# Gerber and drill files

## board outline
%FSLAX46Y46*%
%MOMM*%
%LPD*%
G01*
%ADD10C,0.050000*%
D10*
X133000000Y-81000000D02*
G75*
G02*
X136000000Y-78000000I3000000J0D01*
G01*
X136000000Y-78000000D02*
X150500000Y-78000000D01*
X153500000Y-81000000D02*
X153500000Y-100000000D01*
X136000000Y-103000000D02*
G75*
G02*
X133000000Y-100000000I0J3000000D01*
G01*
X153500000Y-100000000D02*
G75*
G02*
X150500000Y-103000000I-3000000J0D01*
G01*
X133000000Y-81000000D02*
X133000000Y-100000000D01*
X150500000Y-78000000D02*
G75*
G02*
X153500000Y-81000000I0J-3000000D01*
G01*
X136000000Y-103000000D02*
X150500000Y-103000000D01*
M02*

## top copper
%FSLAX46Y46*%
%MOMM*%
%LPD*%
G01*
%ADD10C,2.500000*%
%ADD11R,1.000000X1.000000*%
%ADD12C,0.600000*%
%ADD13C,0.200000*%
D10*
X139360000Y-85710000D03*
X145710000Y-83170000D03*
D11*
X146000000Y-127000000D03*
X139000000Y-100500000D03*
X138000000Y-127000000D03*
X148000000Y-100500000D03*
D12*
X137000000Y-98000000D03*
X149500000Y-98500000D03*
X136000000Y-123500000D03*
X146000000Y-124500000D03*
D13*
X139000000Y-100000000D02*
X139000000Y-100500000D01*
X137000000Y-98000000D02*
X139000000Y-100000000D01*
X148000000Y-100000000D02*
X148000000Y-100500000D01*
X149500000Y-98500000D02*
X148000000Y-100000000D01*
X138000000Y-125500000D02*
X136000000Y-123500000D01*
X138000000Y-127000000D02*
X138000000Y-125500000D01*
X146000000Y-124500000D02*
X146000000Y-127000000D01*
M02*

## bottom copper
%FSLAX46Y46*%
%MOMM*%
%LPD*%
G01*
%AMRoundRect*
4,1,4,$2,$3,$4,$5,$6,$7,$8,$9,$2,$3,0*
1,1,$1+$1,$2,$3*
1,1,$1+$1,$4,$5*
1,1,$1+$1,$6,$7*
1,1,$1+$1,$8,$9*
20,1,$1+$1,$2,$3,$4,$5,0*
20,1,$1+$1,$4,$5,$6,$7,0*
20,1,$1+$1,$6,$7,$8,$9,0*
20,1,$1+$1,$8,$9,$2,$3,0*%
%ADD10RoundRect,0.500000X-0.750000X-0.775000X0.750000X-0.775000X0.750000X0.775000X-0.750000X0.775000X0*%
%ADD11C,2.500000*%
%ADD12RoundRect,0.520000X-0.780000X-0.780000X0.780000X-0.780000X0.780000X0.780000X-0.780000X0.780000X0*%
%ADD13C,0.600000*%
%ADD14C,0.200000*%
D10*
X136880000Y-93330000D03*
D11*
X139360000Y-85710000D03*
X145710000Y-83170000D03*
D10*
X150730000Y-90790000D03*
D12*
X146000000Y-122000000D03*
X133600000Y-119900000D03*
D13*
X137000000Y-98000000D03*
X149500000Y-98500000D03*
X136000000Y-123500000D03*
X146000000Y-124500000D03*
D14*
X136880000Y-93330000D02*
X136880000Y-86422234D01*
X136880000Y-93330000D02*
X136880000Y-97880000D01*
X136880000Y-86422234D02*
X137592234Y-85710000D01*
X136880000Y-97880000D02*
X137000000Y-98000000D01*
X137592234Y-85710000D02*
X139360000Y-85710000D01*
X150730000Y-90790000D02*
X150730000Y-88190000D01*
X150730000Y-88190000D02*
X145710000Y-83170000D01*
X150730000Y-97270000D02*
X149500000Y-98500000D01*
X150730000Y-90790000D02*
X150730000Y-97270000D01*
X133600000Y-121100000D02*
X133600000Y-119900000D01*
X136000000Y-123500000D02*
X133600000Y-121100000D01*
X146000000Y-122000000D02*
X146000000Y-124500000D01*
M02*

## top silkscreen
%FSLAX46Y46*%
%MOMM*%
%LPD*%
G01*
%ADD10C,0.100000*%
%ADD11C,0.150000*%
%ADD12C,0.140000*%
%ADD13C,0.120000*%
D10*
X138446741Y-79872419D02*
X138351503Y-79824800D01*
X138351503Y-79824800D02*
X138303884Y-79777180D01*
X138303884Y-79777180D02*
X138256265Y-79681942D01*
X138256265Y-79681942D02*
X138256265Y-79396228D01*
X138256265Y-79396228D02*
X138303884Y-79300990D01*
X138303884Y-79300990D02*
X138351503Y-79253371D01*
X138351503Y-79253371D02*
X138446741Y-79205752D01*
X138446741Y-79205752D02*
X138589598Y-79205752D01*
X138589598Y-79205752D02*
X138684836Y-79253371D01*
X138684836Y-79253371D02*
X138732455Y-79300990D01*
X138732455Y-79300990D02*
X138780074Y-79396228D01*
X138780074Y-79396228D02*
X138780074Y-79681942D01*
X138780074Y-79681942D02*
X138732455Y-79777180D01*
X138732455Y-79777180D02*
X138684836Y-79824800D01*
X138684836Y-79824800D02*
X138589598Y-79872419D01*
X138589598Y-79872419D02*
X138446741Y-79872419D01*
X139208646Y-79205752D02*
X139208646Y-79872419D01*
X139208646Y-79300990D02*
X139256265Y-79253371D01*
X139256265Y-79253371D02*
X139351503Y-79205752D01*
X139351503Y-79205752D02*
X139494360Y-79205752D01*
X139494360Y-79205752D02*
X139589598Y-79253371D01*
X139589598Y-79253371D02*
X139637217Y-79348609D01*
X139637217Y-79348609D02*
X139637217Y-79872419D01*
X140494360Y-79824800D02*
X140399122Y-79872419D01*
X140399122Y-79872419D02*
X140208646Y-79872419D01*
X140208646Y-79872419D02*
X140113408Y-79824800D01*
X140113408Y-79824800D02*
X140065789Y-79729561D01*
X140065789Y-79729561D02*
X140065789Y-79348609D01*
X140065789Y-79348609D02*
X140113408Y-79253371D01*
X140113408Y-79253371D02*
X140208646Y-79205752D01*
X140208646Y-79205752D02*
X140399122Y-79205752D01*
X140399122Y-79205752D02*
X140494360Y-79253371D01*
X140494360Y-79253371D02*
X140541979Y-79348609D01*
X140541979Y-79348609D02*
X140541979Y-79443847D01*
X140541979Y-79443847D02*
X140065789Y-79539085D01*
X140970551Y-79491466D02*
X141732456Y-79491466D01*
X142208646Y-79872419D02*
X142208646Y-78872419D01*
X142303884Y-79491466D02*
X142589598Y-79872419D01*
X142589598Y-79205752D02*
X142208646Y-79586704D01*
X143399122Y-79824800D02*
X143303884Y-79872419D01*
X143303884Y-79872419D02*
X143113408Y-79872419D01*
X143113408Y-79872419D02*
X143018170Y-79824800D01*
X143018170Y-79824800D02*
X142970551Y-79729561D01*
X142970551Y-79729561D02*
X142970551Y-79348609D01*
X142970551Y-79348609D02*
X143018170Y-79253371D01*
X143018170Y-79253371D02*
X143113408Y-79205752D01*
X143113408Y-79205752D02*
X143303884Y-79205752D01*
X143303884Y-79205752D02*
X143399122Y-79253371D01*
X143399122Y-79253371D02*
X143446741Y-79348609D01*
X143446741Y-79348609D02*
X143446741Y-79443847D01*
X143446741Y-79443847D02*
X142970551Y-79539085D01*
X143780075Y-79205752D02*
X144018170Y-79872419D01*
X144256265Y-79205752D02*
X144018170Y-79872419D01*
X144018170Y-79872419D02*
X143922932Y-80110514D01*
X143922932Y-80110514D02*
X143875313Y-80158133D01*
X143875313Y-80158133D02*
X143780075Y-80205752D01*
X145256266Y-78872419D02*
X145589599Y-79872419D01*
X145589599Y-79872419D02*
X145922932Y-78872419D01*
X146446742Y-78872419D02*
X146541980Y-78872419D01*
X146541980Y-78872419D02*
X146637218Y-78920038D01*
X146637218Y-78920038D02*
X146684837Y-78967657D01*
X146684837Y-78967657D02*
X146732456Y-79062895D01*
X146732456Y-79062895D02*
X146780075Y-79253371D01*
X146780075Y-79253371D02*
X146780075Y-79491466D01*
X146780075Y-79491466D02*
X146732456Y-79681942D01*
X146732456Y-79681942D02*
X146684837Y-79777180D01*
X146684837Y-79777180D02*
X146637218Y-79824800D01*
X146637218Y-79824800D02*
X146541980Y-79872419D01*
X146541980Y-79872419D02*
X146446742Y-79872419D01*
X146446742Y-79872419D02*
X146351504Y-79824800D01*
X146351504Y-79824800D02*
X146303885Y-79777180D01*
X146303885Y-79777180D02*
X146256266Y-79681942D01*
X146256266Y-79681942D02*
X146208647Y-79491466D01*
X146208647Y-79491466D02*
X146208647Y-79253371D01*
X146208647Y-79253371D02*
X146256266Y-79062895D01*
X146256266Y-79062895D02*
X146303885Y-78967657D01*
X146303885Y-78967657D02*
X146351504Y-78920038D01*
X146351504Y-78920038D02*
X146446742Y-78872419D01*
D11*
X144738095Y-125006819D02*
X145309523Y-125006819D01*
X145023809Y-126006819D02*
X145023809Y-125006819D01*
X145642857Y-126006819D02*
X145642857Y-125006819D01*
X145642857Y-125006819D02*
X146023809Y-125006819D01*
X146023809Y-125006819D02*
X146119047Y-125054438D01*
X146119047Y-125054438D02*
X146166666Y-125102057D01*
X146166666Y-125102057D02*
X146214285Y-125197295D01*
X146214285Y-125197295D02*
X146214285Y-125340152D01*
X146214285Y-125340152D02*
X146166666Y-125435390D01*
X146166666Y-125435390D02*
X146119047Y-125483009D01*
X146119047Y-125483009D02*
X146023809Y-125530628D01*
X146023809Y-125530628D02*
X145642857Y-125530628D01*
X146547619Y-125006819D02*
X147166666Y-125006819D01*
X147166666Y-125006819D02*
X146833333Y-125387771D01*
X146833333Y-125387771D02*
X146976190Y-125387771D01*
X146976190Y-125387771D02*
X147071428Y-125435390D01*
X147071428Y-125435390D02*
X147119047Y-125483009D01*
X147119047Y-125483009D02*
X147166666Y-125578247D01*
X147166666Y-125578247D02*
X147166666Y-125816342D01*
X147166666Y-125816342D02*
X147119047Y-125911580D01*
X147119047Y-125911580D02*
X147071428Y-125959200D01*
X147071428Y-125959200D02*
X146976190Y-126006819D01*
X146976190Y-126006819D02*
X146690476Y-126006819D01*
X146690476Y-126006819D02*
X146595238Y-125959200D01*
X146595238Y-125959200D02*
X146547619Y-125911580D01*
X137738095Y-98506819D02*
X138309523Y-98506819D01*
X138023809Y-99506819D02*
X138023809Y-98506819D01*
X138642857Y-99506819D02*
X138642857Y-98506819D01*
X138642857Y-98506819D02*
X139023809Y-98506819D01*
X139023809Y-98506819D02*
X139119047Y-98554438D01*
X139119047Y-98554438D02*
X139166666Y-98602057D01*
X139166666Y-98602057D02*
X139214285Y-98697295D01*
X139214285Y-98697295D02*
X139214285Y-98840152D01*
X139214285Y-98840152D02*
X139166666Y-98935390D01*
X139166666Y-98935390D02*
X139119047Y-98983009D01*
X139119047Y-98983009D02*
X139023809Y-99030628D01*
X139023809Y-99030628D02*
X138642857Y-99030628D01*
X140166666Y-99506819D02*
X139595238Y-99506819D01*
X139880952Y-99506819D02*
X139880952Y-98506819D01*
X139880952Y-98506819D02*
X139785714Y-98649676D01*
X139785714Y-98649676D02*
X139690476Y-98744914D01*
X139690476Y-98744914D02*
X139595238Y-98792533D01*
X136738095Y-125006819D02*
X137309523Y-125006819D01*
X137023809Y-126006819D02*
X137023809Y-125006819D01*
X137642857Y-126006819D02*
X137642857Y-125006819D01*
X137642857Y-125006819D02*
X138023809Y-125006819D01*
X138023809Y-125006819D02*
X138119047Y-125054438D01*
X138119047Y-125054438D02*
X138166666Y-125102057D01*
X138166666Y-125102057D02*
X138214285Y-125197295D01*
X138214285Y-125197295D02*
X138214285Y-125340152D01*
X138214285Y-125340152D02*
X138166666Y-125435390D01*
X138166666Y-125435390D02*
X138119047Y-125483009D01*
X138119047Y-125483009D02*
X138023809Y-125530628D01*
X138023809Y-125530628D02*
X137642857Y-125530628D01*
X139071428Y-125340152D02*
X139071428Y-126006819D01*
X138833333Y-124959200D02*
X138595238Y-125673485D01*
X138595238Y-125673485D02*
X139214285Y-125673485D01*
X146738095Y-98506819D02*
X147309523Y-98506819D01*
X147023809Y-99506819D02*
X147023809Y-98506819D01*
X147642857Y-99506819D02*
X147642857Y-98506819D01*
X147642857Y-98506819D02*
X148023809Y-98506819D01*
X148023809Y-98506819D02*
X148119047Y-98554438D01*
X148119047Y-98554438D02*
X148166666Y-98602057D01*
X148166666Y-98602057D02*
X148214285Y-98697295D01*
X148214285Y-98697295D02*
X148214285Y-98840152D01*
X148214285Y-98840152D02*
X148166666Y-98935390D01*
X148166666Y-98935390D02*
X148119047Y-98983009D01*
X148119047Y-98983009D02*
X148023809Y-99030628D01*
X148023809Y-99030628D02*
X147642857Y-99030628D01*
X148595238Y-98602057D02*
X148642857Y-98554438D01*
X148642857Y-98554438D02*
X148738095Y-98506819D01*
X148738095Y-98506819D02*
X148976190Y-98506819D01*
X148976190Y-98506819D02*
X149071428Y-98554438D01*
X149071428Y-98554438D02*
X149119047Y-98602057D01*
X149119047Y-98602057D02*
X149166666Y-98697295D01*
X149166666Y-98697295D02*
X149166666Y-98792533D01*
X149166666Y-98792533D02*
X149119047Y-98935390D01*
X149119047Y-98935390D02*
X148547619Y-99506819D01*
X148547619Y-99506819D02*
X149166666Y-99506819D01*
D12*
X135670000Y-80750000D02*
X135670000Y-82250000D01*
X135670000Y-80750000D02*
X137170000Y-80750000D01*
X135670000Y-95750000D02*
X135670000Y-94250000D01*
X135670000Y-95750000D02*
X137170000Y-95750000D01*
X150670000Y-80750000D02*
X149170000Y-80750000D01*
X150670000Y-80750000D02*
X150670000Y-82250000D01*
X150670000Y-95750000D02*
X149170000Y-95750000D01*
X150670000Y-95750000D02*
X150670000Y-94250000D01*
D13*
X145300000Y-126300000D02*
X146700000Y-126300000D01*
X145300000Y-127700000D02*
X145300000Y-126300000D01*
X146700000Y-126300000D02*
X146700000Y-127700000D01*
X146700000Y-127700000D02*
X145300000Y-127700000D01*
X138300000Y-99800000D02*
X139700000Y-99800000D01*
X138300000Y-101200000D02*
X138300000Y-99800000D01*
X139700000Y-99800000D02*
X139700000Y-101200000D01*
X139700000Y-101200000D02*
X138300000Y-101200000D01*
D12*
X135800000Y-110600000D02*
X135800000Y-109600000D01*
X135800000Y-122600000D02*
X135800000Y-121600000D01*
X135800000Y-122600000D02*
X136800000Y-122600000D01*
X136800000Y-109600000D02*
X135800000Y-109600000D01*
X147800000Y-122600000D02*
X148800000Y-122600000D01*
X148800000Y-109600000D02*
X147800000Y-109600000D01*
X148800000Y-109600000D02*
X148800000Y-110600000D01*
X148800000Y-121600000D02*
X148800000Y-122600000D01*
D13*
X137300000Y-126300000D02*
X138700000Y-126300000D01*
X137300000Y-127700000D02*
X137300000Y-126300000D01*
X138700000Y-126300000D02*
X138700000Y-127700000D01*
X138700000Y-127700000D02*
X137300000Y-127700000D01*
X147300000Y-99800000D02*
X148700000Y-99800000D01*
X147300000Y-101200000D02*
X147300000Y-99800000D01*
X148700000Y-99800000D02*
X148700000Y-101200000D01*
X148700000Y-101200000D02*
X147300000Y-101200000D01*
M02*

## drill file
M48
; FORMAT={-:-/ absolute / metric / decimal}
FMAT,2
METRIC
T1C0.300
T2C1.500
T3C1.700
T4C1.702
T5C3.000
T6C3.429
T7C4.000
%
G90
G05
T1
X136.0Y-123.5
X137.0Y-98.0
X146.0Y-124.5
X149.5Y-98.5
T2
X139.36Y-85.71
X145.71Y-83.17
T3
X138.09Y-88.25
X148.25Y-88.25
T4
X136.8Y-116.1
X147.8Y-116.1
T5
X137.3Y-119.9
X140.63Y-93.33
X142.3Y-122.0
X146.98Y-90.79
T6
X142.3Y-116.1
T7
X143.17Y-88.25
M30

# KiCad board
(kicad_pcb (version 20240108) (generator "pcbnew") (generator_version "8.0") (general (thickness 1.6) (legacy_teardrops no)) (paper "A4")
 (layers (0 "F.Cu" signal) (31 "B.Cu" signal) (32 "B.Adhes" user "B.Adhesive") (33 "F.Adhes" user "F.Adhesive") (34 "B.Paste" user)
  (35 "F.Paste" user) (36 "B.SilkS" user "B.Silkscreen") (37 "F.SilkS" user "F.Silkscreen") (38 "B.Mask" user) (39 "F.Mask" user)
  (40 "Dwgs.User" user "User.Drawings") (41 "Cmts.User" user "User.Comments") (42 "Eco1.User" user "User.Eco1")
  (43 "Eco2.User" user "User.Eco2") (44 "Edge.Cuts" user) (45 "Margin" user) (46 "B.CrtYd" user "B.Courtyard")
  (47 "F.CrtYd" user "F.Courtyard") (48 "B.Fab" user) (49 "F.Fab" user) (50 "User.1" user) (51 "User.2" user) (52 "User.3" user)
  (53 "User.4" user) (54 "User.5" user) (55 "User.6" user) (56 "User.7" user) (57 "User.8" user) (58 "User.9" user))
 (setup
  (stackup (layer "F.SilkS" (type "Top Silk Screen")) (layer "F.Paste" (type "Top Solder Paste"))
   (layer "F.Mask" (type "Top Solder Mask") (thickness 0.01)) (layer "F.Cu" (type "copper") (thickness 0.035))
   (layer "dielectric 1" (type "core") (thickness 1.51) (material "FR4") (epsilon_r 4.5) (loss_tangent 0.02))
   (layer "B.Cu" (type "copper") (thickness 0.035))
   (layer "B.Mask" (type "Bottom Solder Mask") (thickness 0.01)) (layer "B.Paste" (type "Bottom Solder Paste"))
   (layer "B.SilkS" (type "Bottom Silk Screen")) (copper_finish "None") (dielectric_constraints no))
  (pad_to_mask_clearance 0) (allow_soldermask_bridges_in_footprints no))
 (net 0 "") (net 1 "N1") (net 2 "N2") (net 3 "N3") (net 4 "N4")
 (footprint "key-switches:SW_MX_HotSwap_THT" (layer "F.Cu") (at 143.17 88.25)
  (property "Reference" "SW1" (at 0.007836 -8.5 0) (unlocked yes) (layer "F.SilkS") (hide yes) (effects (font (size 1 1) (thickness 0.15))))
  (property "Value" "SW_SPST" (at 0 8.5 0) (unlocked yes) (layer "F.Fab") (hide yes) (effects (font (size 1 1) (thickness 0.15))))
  (fp_line (start -7.5 -7.5) (end -7.5 -6) (stroke (width 0.14) (type solid)) (layer "F.SilkS"))
  (fp_line (start -7.5 -7.5) (end -6 -7.5) (stroke (width 0.14) (type solid)) (layer "F.SilkS"))
  (fp_line (start -7.5 7.5) (end -7.5 6) (stroke (width 0.14) (type solid)) (layer "F.SilkS"))
  (fp_line (start -7.5 7.5) (end -6 7.5) (stroke (width 0.14) (type solid)) (layer "F.SilkS"))
  (fp_line (start 7.5 -7.5) (end 6 -7.5) (stroke (width 0.14) (type solid)) (layer "F.SilkS"))
  (fp_line (start 7.5 -7.5) (end 7.5 -6) (stroke (width 0.14) (type solid)) (layer "F.SilkS"))
  (fp_line (start 7.5 7.5) (end 6 7.5) (stroke (width 0.14) (type solid)) (layer "F.SilkS"))
  (fp_line (start 7.5 7.5) (end 7.5 6) (stroke (width 0.14) (type solid)) (layer "F.SilkS"))
  (pad "" np_thru_hole circle (at -5.08 0) (size 1.7 1.7) (drill 1.7) (layers "*.Mask"))
  (pad "" np_thru_hole circle (at -2.54 5.08) (size 3 3) (drill 3) (layers "*.Mask"))
  (pad "" np_thru_hole circle (at 0 0) (size 4 4) (drill 4) (layers "*.Mask"))
  (pad "" np_thru_hole circle (at 3.81 2.54) (size 3 3) (drill 3) (layers "*.Mask"))
  (pad "" np_thru_hole circle (at 5.08 0) (size 1.7 1.7) (drill 1.7) (layers "*.Mask"))
  (pad "1" smd roundrect (at -6.29 5.08) (size 2.5 2.55) (layers "B.Cu" "B.Paste" "B.Mask") (roundrect_rratio 0.2) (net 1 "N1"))
  (pad "1" thru_hole circle (at -3.81 -2.54) (size 2.5 2.5) (drill 1.5) (layers "*.Cu" "*.Mask") (remove_unused_layers no) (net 1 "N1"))
  (pad "2" thru_hole circle (at 2.54 -5.08) (size 2.5 2.5) (drill 1.5) (layers "*.Cu" "*.Mask") (remove_unused_layers no) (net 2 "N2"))
  (pad "2" smd roundrect (at 7.56 2.54) (size 2.5 2.55) (layers "B.Cu" "B.Paste" "B.Mask") (roundrect_rratio 0.2) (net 2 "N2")))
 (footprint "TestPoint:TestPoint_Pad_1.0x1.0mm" (layer "F.Cu") (at 146 127)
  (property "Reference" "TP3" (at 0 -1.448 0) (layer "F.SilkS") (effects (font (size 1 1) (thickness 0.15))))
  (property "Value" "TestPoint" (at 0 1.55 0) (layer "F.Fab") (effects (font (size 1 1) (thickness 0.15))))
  (fp_line (start -0.7 -0.7) (end 0.7 -0.7) (stroke (width 0.12) (type solid)) (layer "F.SilkS"))
  (fp_line (start -0.7 0.7) (end -0.7 -0.7) (stroke (width 0.12) (type solid)) (layer "F.SilkS"))
  (fp_line (start 0.7 -0.7) (end 0.7 0.7) (stroke (width 0.12) (type solid)) (layer "F.SilkS"))
  (fp_line (start 0.7 0.7) (end -0.7 0.7) (stroke (width 0.12) (type solid)) (layer "F.SilkS"))
  (pad "1" smd rect (at 0 0) (size 1 1) (layers "F.Cu" "F.Mask") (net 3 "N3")))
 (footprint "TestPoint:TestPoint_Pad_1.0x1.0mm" (layer "F.Cu") (at 139 100.5)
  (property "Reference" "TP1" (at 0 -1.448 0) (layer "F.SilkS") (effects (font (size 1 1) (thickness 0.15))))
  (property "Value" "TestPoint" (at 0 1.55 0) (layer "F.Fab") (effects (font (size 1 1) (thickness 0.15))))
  (fp_line (start -0.7 -0.7) (end 0.7 -0.7) (stroke (width 0.12) (type solid)) (layer "F.SilkS"))
  (fp_line (start -0.7 0.7) (end -0.7 -0.7) (stroke (width 0.12) (type solid)) (layer "F.SilkS"))
  (fp_line (start 0.7 -0.7) (end 0.7 0.7) (stroke (width 0.12) (type solid)) (layer "F.SilkS"))
  (fp_line (start 0.7 0.7) (end -0.7 0.7) (stroke (width 0.12) (type solid)) (layer "F.SilkS"))
  (pad "1" smd rect (at 0 0) (size 1 1) (layers "F.Cu" "F.Mask") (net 1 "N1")))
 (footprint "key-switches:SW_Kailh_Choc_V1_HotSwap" (layer "F.Cu") (at 142.3 116.1)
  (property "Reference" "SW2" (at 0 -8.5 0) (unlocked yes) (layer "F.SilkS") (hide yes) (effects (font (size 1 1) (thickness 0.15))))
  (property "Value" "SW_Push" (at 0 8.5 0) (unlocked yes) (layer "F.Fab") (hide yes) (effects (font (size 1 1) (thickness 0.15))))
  (fp_line (start -6.5 -5.5) (end -6.5 -6.5) (stroke (width 0.14) (type solid)) (layer "F.SilkS"))
  (fp_line (start -6.5 6.5) (end -6.5 5.5) (stroke (width 0.14) (type solid)) (layer "F.SilkS"))
  (fp_line (start -6.5 6.5) (end -5.5 6.5) (stroke (width 0.14) (type solid)) (layer "F.SilkS"))
  (fp_line (start -5.5 -6.5) (end -6.5 -6.5) (stroke (width 0.14) (type solid)) (layer "F.SilkS"))
  (fp_line (start 5.5 6.5) (end 6.5 6.5) (stroke (width 0.14) (type solid)) (layer "F.SilkS"))
  (fp_line (start 6.5 -6.5) (end 5.5 -6.5) (stroke (width 0.14) (type solid)) (layer "F.SilkS"))
  (fp_line (start 6.5 -6.5) (end 6.5 -5.5) (stroke (width 0.14) (type solid)) (layer "F.SilkS"))
  (fp_line (start 6.5 5.5) (end 6.5 6.5) (stroke (width 0.14) (type solid)) (layer "F.SilkS"))
  (pad "" np_thru_hole circle (at -5.5 0) (size 1.7018 1.7018) (drill 1.7018) (layers "*.Cu" "*.Mask"))
  (pad "" np_thru_hole circle (at -5 3.8) (size 3 3) (drill 3) (layers "F&B.Cu" "*.Mask"))
  (pad "" np_thru_hole circle (at 0 0) (size 3.429 3.429) (drill 3.429) (layers "*.Cu" "*.Mask"))
  (pad "" np_thru_hole circle (at 0 5.9) (size 3 3) (drill 3) (layers "F&B.Cu" "*.Mask"))
  (pad "" np_thru_hole circle (at 5.5 0) (size 1.7018 1.7018) (drill 1.7018) (layers "*.Cu" "*.Mask"))
  (pad "1" smd roundrect (at 3.7 5.9) (size 2.6 2.6) (layers "B.Cu" "B.Paste" "B.Mask") (roundrect_rratio 0.2) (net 3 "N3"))
  (pad "2" smd roundrect (at -8.7 3.8) (size 2.6 2.6) (layers "B.Cu" "B.Paste" "B.Mask") (roundrect_rratio 0.2) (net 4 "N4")))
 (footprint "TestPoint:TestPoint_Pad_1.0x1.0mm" (layer "F.Cu") (at 138 127)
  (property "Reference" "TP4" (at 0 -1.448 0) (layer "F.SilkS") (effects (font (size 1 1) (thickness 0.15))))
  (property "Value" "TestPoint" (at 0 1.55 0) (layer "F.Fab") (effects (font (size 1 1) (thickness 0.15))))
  (fp_line (start -0.7 -0.7) (end 0.7 -0.7) (stroke (width 0.12) (type solid)) (layer "F.SilkS"))
  (fp_line (start -0.7 0.7) (end -0.7 -0.7) (stroke (width 0.12) (type solid)) (layer "F.SilkS"))
  (fp_line (start 0.7 -0.7) (end 0.7 0.7) (stroke (width 0.12) (type solid)) (layer "F.SilkS"))
  (fp_line (start 0.7 0.7) (end -0.7 0.7) (stroke (width 0.12) (type solid)) (layer "F.SilkS"))
  (pad "1" smd rect (at 0 0) (size 1 1) (layers "F.Cu" "F.Mask") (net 4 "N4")))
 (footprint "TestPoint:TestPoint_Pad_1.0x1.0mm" (layer "F.Cu") (at 148 100.5)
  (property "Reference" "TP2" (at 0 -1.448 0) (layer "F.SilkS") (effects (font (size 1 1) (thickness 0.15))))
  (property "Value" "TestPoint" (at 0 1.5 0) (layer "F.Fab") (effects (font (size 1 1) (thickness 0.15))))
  (fp_line (start -0.7 -0.7) (end 0.7 -0.7) (stroke (width 0.12) (type solid)) (layer "F.SilkS"))
  (fp_line (start -0.7 0.7) (end -0.7 -0.7) (stroke (width 0.12) (type solid)) (layer "F.SilkS"))
  (fp_line (start 0.7 -0.7) (end 0.7 0.7) (stroke (width 0.12) (type solid)) (layer "F.SilkS"))
  (fp_line (start 0.7 0.7) (end -0.7 0.7) (stroke (width 0.12) (type solid)) (layer "F.SilkS"))
  (pad "1" smd rect (at 0 0) (size 1 1) (layers "F.Cu" "F.Mask") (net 2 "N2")))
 (gr_arc (start 133 81) (mid 133.87868 78.87868) (end 136 78) (stroke (width 0.05) (type default)) (layer "Edge.Cuts"))
 (gr_line (start 136 78) (end 150.5 78) (stroke (width 0.05) (type default)) (layer "Edge.Cuts"))
 (gr_line (start 153.5 81) (end 153.5 100) (stroke (width 0.05) (type default)) (layer "Edge.Cuts"))
 (gr_arc (start 136 103) (mid 133.87868 102.12132) (end 133 100) (stroke (width 0.05) (type default)) (layer "Edge.Cuts"))
 (gr_arc (start 153.5 100) (mid 152.62132 102.12132) (end 150.5 103) (stroke (width 0.05) (type default)) (layer "Edge.Cuts"))
 (gr_line (start 133 81) (end 133 100) (stroke (width 0.05) (type default)) (layer "Edge.Cuts"))
 (gr_arc (start 150.5 78) (mid 152.62132 78.87868) (end 153.5 81) (stroke (width 0.05) (type default)) (layer "Edge.Cuts"))
 (gr_line (start 136 103) (end 150.5 103) (stroke (width 0.05) (type default)) (layer "Edge.Cuts"))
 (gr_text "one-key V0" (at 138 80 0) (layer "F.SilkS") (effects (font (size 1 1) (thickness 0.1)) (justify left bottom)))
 (segment (start 139 100) (end 139 100.5) (width 0.2) (layer "F.Cu") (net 1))
 (segment (start 137 98) (end 139 100) (width 0.2) (layer "F.Cu") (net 1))
 (via (at 137 98) (size 0.6) (drill 0.3) (layers "F.Cu" "B.Cu") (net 1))
 (segment (start 136.88 93.33) (end 136.88 86.422234) (width 0.2) (layer "B.Cu") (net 1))
 (segment (start 136.88 93.33) (end 136.88 97.88) (width 0.2) (layer "B.Cu") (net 1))
 (segment (start 136.88 86.422234) (end 137.592234 85.71) (width 0.2) (layer "B.Cu") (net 1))
 (segment (start 136.88 97.88) (end 137 98) (width 0.2) (layer "B.Cu") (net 1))
 (segment (start 137.592234 85.71) (end 139.36 85.71) (width 0.2) (layer "B.Cu") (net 1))
 (segment (start 148 100) (end 148 100.5) (width 0.2) (layer "F.Cu") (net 2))
 (segment (start 149.5 98.5) (end 148 100) (width 0.2) (layer "F.Cu") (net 2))
 (via (at 149.5 98.5) (size 0.6) (drill 0.3) (layers "F.Cu" "B.Cu") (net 2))
 (segment (start 150.73 90.79) (end 150.73 88.19) (width 0.2) (layer "B.Cu") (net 2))
 (segment (start 150.73 88.19) (end 145.71 83.17) (width 0.2) (layer "B.Cu") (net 2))
 (segment (start 150.73 97.27) (end 149.5 98.5) (width 0.2) (layer "B.Cu") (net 2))
 (segment (start 150.73 90.79) (end 150.73 97.27) (width 0.2) (layer "B.Cu") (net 2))
 (segment (start 138 125.5) (end 136 123.5) (width 0.2) (layer "F.Cu") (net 4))
 (segment (start 138 127) (end 138 125.5) (width 0.2) (layer "F.Cu") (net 4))
 (via (at 136 123.5) (size 0.6) (drill 0.3) (layers "F.Cu" "B.Cu") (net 4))
 (segment (start 133.6 121.1) (end 133.6 119.9) (width 0.2) (layer "B.Cu") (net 4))
 (segment (start 136 123.5) (end 133.6 121.1) (width 0.2) (layer "B.Cu") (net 4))
 (segment (start 146 124.5) (end 146 127) (width 0.2) (layer "F.Cu") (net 3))
 (via (at 146 124.5) (size 0.6) (drill 0.3) (layers "F.Cu" "B.Cu") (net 3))
 (segment (start 146 122) (end 146 124.5) (width 0.2) (layer "B.Cu") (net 3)))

